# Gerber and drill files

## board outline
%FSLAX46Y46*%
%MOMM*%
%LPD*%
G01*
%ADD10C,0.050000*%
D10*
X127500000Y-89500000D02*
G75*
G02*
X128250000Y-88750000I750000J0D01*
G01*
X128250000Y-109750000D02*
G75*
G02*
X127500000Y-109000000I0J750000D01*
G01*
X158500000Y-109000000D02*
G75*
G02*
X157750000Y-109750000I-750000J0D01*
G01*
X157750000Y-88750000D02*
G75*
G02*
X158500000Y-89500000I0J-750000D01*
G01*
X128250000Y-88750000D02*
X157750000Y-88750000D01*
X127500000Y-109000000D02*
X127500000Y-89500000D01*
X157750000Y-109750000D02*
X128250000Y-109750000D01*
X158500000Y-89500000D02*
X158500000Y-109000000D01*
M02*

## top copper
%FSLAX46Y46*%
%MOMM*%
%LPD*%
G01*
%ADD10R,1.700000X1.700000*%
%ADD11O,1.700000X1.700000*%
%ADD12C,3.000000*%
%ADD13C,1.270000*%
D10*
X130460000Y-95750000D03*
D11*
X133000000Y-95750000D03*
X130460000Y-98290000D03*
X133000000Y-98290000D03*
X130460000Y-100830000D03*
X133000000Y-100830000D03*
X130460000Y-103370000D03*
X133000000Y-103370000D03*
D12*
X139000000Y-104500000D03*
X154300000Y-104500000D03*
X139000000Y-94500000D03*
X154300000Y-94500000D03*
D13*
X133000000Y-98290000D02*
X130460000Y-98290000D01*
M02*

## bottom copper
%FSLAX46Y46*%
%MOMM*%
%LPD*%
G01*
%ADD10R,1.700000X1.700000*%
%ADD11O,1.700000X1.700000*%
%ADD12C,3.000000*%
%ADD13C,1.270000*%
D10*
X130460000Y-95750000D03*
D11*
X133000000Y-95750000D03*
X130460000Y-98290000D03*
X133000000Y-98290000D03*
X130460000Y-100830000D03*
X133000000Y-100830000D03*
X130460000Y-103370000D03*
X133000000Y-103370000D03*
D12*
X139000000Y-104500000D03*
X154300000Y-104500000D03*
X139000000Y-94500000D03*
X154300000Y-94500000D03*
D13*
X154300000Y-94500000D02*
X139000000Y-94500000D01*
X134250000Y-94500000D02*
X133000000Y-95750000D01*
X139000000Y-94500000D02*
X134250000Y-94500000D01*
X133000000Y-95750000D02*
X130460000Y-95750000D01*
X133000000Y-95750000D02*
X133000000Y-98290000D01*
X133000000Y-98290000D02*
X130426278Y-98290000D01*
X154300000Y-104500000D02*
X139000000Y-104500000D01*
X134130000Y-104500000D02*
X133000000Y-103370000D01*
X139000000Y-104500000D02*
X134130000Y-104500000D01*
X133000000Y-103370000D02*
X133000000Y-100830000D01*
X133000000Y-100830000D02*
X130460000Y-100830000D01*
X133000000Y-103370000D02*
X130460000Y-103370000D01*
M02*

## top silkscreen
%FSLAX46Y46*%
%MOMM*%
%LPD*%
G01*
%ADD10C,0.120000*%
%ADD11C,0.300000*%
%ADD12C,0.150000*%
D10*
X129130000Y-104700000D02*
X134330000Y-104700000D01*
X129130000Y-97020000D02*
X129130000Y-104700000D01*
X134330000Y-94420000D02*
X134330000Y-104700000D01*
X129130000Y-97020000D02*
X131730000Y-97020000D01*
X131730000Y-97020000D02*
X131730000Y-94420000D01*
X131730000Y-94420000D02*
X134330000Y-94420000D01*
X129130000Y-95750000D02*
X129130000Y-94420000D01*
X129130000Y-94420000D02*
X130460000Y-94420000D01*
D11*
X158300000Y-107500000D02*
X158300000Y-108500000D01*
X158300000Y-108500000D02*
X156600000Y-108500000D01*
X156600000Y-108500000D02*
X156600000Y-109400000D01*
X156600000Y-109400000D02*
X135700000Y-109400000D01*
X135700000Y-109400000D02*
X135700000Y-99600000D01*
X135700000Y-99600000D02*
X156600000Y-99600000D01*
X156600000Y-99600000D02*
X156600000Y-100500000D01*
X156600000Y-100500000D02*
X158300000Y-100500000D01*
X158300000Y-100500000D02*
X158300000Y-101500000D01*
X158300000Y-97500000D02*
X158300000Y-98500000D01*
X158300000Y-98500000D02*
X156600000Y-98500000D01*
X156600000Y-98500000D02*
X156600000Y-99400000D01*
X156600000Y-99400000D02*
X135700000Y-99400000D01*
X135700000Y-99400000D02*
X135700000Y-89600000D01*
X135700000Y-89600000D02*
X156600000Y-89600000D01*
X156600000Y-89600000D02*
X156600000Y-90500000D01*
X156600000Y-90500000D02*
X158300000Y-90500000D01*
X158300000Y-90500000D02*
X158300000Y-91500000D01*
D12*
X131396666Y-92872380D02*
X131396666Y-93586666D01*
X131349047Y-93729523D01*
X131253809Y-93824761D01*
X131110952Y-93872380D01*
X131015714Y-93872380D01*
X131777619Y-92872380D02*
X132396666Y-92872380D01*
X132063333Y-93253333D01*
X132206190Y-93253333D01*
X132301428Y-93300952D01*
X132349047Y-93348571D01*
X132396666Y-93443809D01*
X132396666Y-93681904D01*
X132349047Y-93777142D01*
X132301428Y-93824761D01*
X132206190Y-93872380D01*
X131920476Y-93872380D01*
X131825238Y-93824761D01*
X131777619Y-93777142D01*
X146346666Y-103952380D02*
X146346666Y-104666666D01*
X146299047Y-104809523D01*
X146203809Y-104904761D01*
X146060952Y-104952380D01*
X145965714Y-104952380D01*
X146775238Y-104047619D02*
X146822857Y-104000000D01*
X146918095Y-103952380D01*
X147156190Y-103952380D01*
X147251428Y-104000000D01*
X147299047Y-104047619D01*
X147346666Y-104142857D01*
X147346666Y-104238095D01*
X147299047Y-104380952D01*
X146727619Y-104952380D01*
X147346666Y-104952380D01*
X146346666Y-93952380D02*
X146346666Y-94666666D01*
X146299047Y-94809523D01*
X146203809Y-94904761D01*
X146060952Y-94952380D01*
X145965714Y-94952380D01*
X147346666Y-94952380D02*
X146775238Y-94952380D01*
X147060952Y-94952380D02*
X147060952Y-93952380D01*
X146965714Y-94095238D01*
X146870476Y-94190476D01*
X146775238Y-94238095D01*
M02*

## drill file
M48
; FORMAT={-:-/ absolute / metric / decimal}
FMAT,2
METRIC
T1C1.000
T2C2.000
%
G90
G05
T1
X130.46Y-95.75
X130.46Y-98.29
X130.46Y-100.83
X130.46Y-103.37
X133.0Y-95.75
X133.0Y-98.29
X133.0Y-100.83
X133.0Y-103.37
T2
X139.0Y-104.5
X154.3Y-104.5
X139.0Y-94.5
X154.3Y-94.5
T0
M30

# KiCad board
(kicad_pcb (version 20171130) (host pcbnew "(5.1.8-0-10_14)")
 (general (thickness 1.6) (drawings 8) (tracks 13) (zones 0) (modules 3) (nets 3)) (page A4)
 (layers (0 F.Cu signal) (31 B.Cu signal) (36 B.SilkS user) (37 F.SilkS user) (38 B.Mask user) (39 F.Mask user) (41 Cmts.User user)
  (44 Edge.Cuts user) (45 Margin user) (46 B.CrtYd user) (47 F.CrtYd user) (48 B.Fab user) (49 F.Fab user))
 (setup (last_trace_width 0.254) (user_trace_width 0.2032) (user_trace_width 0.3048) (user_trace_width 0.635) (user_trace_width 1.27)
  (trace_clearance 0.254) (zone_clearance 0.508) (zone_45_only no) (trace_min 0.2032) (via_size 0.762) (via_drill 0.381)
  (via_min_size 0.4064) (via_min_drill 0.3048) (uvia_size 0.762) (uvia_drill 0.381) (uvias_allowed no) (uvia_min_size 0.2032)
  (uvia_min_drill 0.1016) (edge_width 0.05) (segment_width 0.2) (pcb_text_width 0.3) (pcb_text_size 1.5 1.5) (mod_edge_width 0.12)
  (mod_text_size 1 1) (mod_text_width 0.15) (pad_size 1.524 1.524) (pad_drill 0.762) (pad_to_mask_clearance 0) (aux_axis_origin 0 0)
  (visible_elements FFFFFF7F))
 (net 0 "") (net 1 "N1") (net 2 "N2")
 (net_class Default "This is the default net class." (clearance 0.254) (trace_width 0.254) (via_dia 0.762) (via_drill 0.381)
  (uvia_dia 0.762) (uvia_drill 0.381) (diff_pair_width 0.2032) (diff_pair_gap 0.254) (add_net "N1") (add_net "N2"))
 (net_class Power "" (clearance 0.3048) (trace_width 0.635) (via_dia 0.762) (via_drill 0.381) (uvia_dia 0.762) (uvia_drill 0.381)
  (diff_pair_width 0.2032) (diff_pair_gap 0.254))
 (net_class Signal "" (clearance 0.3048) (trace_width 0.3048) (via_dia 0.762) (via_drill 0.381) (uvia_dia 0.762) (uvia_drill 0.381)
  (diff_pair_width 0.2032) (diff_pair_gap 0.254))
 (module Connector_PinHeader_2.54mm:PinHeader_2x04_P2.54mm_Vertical (layer F.Cu) (at 130.46 95.75)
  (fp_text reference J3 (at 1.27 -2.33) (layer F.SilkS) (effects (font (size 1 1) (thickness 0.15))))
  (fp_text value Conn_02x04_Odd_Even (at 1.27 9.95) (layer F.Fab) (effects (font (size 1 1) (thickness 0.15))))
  (fp_line (start -1.33 8.95) (end 3.87 8.95) (layer F.SilkS) (width 0.12))
  (fp_line (start -1.33 1.27) (end -1.33 8.95) (layer F.SilkS) (width 0.12))
  (fp_line (start 3.87 -1.33) (end 3.87 8.95) (layer F.SilkS) (width 0.12))
  (fp_line (start -1.33 1.27) (end 1.27 1.27) (layer F.SilkS) (width 0.12))
  (fp_line (start 1.27 1.27) (end 1.27 -1.33) (layer F.SilkS) (width 0.12))
  (fp_line (start 1.27 -1.33) (end 3.87 -1.33) (layer F.SilkS) (width 0.12))
  (fp_line (start -1.33 0) (end -1.33 -1.33) (layer F.SilkS) (width 0.12))
  (fp_line (start -1.33 -1.33) (end 0 -1.33) (layer F.SilkS) (width 0.12))
  (pad 1 thru_hole rect (at 0 0) (size 1.7 1.7) (drill 1) (layers *.Cu *.Mask) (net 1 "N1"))
  (pad 2 thru_hole oval (at 2.54 0) (size 1.7 1.7) (drill 1) (layers *.Cu *.Mask) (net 1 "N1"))
  (pad 3 thru_hole oval (at 0 2.54) (size 1.7 1.7) (drill 1) (layers *.Cu *.Mask) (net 1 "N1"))
  (pad 4 thru_hole oval (at 2.54 2.54) (size 1.7 1.7) (drill 1) (layers *.Cu *.Mask) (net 1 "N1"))
  (pad 5 thru_hole oval (at 0 5.08) (size 1.7 1.7) (drill 1) (layers *.Cu *.Mask) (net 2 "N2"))
  (pad 6 thru_hole oval (at 2.54 5.08) (size 1.7 1.7) (drill 1) (layers *.Cu *.Mask) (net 2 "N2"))
  (pad 7 thru_hole oval (at 0 7.62) (size 1.7 1.7) (drill 1) (layers *.Cu *.Mask) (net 2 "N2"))
  (pad 8 thru_hole oval (at 2.54 7.62) (size 1.7 1.7) (drill 1) (layers *.Cu *.Mask) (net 2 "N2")))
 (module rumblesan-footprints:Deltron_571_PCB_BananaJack (layer F.Cu) (at 154.3 104.5)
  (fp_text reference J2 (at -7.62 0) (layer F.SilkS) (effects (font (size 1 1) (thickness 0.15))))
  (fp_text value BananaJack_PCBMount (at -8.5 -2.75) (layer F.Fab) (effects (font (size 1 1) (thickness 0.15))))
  (fp_line (start 4 3) (end 4 4) (layer F.SilkS) (width 0.3))
  (fp_line (start 4 4) (end 2.3 4) (layer F.SilkS) (width 0.3))
  (fp_line (start 2.3 4) (end 2.3 4.9) (layer F.SilkS) (width 0.3))
  (fp_line (start 2.3 4.9) (end -18.6 4.9) (layer F.SilkS) (width 0.3))
  (fp_line (start -18.6 4.9) (end -18.6 -4.9) (layer F.SilkS) (width 0.3))
  (fp_line (start -18.6 -4.9) (end 2.3 -4.9) (layer F.SilkS) (width 0.3))
  (fp_line (start 2.3 -4.9) (end 2.3 -4) (layer F.SilkS) (width 0.3))
  (fp_line (start 2.3 -4) (end 4 -4) (layer F.SilkS) (width 0.3))
  (fp_line (start 4 -4) (end 4 -3) (layer F.SilkS) (width 0.3))
  (pad 1 thru_hole circle (at -15.3 0) (size 3 3) (drill 2) (layers *.Cu *.Mask) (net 2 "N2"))
  (pad 1 thru_hole circle (at 0 0) (size 3 3) (drill 2) (layers *.Cu *.Mask) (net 2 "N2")))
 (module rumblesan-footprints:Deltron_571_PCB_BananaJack (layer F.Cu) (at 154.3 94.5)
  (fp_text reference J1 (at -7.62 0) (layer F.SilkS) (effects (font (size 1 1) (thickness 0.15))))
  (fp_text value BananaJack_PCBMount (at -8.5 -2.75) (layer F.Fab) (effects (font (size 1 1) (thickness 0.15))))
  (fp_line (start 4 3) (end 4 4) (layer F.SilkS) (width 0.3))
  (fp_line (start 4 4) (end 2.3 4) (layer F.SilkS) (width 0.3))
  (fp_line (start 2.3 4) (end 2.3 4.9) (layer F.SilkS) (width 0.3))
  (fp_line (start 2.3 4.9) (end -18.6 4.9) (layer F.SilkS) (width 0.3))
  (fp_line (start -18.6 4.9) (end -18.6 -4.9) (layer F.SilkS) (width 0.3))
  (fp_line (start -18.6 -4.9) (end 2.3 -4.9) (layer F.SilkS) (width 0.3))
  (fp_line (start 2.3 -4.9) (end 2.3 -4) (layer F.SilkS) (width 0.3))
  (fp_line (start 2.3 -4) (end 4 -4) (layer F.SilkS) (width 0.3))
  (fp_line (start 4 -4) (end 4 -3) (layer F.SilkS) (width 0.3))
  (pad 1 thru_hole circle (at -15.3 0) (size 3 3) (drill 2) (layers *.Cu *.Mask) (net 1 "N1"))
  (pad 1 thru_hole circle (at 0 0) (size 3 3) (drill 2) (layers *.Cu *.Mask) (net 1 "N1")))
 (gr_arc (start 128.25 89.5) (end 128.25 88.75) (angle -90) (layer Edge.Cuts) (width 0.05))
 (gr_arc (start 128.25 109) (end 127.5 109) (angle -90) (layer Edge.Cuts) (width 0.05))
 (gr_arc (start 157.75 109) (end 157.75 109.75) (angle -90) (layer Edge.Cuts) (width 0.05))
 (gr_arc (start 157.75 89.5) (end 158.5 89.5) (angle -90) (layer Edge.Cuts) (width 0.05))
 (gr_line (start 128.25 88.75) (end 157.75 88.75) (layer Edge.Cuts) (width 0.05))
 (gr_line (start 127.5 109) (end 127.5 89.5) (layer Edge.Cuts) (width 0.05))
 (gr_line (start 157.75 109.75) (end 128.25 109.75) (layer Edge.Cuts) (width 0.05))
 (gr_line (start 158.5 89.5) (end 158.5 109) (layer Edge.Cuts) (width 0.05))
 (segment (start 133 98.29) (end 130.46 98.29) (width 1.27) (layer F.Cu) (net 1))
 (segment (start 154.3 94.5) (end 139 94.5) (width 1.27) (layer B.Cu) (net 1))
 (segment (start 134.25 94.5) (end 133 95.75) (width 1.27) (layer B.Cu) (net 1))
 (segment (start 139 94.5) (end 134.25 94.5) (width 1.27) (layer B.Cu) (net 1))
 (segment (start 133 95.75) (end 130.46 95.75) (width 1.27) (layer B.Cu) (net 1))
 (segment (start 133 95.75) (end 133 98.29) (width 1.27) (layer B.Cu) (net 1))
 (segment (start 133 98.29) (end 130.426278 98.29) (width 1.27) (layer B.Cu) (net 1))
 (segment (start 154.3 104.5) (end 139 104.5) (width 1.27) (layer B.Cu) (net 2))
 (segment (start 134.13 104.5) (end 133 103.37) (width 1.27) (layer B.Cu) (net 2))
 (segment (start 139 104.5) (end 134.13 104.5) (width 1.27) (layer B.Cu) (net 2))
 (segment (start 133 103.37) (end 133 100.83) (width 1.27) (layer B.Cu) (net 2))
 (segment (start 133 100.83) (end 130.46 100.83) (width 1.27) (layer B.Cu) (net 2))
 (segment (start 133 103.37) (end 130.46 103.37) (width 1.27) (layer B.Cu) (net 2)))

